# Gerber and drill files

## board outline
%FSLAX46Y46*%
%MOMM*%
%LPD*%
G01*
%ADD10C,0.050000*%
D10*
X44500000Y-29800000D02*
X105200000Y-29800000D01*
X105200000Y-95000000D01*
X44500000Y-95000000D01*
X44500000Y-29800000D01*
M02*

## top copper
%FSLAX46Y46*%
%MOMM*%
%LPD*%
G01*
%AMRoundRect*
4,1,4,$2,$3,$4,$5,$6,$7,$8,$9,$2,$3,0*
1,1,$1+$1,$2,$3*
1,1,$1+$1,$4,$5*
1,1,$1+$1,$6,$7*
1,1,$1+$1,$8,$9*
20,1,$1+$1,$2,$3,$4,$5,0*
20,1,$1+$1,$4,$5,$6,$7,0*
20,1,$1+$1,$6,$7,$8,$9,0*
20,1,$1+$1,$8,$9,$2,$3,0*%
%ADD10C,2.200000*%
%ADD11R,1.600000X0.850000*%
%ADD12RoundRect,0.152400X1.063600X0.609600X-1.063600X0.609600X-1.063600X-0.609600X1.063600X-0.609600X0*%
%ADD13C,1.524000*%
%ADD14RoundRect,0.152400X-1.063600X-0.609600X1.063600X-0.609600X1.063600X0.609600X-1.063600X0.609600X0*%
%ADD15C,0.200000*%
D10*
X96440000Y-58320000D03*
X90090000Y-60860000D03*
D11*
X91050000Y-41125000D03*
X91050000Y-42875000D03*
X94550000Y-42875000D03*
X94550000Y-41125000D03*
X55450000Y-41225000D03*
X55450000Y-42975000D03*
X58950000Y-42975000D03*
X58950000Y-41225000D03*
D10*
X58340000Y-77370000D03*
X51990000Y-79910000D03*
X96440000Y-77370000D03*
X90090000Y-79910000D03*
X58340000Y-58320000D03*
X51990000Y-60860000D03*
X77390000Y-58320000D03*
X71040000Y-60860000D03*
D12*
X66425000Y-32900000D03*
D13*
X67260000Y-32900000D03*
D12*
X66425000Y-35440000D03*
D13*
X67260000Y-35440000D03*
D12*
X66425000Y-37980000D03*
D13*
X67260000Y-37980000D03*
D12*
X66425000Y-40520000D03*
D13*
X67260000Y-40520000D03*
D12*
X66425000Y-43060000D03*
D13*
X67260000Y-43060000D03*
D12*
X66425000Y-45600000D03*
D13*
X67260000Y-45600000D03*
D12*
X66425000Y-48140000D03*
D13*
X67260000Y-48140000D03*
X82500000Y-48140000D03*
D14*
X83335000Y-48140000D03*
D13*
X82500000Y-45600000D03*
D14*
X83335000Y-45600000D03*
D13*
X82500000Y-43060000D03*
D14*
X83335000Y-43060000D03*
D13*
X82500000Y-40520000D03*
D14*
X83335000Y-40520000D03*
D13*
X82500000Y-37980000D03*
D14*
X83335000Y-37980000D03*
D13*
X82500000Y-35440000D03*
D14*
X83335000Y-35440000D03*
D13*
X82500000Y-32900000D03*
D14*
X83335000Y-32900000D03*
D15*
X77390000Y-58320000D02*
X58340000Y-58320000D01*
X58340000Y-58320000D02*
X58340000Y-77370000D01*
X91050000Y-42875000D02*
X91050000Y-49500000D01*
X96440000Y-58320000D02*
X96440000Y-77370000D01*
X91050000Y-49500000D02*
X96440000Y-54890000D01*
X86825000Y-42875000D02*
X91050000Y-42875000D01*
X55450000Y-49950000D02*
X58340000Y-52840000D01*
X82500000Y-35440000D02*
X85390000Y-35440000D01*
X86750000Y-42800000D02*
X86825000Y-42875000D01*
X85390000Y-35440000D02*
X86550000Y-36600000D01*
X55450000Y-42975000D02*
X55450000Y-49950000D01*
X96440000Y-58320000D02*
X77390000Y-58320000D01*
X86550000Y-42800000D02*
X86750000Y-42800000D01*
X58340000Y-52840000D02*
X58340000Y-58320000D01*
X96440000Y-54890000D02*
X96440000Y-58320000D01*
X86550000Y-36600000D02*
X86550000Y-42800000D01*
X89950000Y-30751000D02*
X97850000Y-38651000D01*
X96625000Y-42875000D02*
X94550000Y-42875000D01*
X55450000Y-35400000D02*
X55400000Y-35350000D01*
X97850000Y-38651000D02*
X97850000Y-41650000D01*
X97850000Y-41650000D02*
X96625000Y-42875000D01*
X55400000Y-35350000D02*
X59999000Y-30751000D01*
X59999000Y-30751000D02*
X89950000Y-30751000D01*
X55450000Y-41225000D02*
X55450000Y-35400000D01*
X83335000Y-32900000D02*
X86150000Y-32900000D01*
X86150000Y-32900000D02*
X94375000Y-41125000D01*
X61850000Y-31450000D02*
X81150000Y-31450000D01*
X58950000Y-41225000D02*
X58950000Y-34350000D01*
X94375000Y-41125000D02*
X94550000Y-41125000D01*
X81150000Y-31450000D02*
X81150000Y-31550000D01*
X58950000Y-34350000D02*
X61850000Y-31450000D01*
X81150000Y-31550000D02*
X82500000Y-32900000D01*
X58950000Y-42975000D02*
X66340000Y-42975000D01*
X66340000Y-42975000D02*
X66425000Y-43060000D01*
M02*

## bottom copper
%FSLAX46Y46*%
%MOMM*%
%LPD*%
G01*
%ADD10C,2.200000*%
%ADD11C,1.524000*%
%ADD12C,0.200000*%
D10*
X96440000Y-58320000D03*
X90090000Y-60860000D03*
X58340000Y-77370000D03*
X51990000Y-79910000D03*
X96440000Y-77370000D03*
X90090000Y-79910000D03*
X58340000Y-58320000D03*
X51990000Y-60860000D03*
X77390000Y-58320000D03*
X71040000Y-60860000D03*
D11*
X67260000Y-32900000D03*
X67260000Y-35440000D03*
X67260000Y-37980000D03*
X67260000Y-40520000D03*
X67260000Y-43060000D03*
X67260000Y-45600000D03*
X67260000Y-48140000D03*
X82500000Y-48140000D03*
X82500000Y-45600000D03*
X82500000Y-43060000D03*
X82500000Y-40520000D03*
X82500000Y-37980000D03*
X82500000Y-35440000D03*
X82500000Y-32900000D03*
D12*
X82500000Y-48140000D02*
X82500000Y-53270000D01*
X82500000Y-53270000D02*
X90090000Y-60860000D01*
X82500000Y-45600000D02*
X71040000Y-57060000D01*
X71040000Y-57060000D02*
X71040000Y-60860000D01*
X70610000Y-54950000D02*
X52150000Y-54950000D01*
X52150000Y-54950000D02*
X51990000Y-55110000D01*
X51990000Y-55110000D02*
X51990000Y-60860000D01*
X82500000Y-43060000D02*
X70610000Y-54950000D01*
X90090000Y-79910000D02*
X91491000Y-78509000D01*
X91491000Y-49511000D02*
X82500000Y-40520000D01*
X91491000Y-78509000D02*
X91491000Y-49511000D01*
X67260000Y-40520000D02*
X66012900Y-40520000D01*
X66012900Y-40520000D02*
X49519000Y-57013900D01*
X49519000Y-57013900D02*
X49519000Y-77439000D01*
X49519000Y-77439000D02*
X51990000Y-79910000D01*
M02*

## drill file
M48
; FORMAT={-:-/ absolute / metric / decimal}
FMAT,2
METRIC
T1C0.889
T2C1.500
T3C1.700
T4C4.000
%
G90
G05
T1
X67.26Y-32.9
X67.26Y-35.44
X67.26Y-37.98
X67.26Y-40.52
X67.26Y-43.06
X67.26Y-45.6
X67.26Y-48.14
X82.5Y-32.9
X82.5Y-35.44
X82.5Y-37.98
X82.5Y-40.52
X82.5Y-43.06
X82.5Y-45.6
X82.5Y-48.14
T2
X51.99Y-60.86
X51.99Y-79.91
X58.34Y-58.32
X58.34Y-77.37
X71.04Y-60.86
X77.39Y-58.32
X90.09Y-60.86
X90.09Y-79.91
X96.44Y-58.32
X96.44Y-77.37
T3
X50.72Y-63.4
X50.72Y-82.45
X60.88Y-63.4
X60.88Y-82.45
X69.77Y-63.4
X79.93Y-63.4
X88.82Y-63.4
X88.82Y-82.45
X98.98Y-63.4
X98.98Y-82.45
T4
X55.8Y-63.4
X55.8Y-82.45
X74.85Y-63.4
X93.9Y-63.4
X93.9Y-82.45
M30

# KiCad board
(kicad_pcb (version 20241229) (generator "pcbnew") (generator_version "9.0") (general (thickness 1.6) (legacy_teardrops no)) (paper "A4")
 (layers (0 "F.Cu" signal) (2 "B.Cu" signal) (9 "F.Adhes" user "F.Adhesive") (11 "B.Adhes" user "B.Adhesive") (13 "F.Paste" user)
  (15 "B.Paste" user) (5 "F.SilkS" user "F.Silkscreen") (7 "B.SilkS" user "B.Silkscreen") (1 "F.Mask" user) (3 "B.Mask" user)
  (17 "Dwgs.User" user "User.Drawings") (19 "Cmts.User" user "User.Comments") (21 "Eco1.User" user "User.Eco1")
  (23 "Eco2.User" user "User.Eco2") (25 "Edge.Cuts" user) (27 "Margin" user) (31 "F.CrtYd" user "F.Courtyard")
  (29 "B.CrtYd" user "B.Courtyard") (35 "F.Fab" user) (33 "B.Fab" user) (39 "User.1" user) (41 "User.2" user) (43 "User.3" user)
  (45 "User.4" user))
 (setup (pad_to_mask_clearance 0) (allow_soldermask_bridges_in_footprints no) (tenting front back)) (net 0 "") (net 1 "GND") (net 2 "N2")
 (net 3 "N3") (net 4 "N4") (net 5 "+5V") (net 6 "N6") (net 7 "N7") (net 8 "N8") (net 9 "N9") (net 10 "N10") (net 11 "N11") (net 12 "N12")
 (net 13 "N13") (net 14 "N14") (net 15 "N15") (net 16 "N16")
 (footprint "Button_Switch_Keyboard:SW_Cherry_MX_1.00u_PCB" (layer "F.Cu") (at 96.44 58.32)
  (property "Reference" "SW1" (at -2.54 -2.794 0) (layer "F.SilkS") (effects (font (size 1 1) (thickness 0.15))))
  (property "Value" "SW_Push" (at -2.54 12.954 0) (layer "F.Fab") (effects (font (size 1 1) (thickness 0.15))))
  (pad "" np_thru_hole circle (at -7.62 5.08) (size 1.7 1.7) (drill 1.7) (layers "*.Cu" "*.Mask"))
  (pad "" np_thru_hole circle (at -2.54 5.08) (size 4 4) (drill 4) (layers "*.Cu" "*.Mask"))
  (pad "" np_thru_hole circle (at 2.54 5.08) (size 1.7 1.7) (drill 1.7) (layers "*.Cu" "*.Mask"))
  (pad "1" thru_hole circle (at 0 0) (size 2.2 2.2) (drill 1.5) (layers "*.Cu" "*.Mask") (remove_unused_layers no) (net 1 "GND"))
  (pad "2" thru_hole circle (at -6.35 2.54) (size 2.2 2.2) (drill 1.5) (layers "*.Cu" "*.Mask") (remove_unused_layers no) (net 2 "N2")))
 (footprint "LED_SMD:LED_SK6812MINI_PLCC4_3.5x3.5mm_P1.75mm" (layer "F.Cu") (at 92.8 42)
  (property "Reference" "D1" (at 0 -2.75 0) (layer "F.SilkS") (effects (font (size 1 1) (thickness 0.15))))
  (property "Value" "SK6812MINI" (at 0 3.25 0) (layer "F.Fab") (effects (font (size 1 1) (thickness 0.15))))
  (pad "1" smd rect (at -1.75 -0.875) (size 1.6 0.85) (layers "F.Cu" "F.Mask" "F.Paste") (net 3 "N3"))
  (pad "2" smd rect (at -1.75 0.875) (size 1.6 0.85) (layers "F.Cu" "F.Mask" "F.Paste") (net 1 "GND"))
  (pad "3" smd rect (at 1.75 0.875) (size 1.6 0.85) (layers "F.Cu" "F.Mask" "F.Paste") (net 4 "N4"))
  (pad "4" smd rect (at 1.75 -0.875) (size 1.6 0.85) (layers "F.Cu" "F.Mask" "F.Paste") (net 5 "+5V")))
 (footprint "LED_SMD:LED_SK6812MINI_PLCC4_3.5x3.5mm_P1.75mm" (layer "F.Cu") (at 57.2 42.1)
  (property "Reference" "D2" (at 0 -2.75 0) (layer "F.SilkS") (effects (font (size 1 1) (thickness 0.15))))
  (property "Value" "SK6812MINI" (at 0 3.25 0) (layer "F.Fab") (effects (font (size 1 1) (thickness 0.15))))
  (pad "1" smd rect (at -1.75 -0.875) (size 1.6 0.85) (layers "F.Cu" "F.Mask" "F.Paste") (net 4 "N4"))
  (pad "2" smd rect (at -1.75 0.875) (size 1.6 0.85) (layers "F.Cu" "F.Mask" "F.Paste") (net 1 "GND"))
  (pad "3" smd rect (at 1.75 0.875) (size 1.6 0.85) (layers "F.Cu" "F.Mask" "F.Paste") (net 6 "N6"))
  (pad "4" smd rect (at 1.75 -0.875) (size 1.6 0.85) (layers "F.Cu" "F.Mask" "F.Paste") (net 5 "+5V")))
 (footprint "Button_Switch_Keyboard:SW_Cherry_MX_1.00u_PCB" (layer "F.Cu") (at 58.34 77.37)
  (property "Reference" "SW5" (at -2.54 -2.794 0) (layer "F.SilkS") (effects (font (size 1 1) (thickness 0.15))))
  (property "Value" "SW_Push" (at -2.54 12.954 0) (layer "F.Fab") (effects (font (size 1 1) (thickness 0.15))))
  (pad "" np_thru_hole circle (at -7.62 5.08) (size 1.7 1.7) (drill 1.7) (layers "*.Cu" "*.Mask"))
  (pad "" np_thru_hole circle (at -2.54 5.08) (size 4 4) (drill 4) (layers "*.Cu" "*.Mask"))
  (pad "" np_thru_hole circle (at 2.54 5.08) (size 1.7 1.7) (drill 1.7) (layers "*.Cu" "*.Mask"))
  (pad "1" thru_hole circle (at 0 0) (size 2.2 2.2) (drill 1.5) (layers "*.Cu" "*.Mask") (remove_unused_layers no) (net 1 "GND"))
  (pad "2" thru_hole circle (at -6.35 2.54) (size 2.2 2.2) (drill 1.5) (layers "*.Cu" "*.Mask") (remove_unused_layers no) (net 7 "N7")))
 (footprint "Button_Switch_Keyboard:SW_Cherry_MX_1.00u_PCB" (layer "F.Cu") (at 96.44 77.37)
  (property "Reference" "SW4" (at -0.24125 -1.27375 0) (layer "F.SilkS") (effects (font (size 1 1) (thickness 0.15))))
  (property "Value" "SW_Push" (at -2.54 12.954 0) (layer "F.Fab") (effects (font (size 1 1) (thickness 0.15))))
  (pad "" np_thru_hole circle (at -7.62 5.08) (size 1.7 1.7) (drill 1.7) (layers "*.Cu" "*.Mask"))
  (pad "" np_thru_hole circle (at -2.54 5.08) (size 4 4) (drill 4) (layers "*.Cu" "*.Mask"))
  (pad "" np_thru_hole circle (at 2.54 5.08) (size 1.7 1.7) (drill 1.7) (layers "*.Cu" "*.Mask"))
  (pad "1" thru_hole circle (at 0 0) (size 2.2 2.2) (drill 1.5) (layers "*.Cu" "*.Mask") (remove_unused_layers no) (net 1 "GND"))
  (pad "2" thru_hole circle (at -6.35 2.54) (size 2.2 2.2) (drill 1.5) (layers "*.Cu" "*.Mask") (remove_unused_layers no) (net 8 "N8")))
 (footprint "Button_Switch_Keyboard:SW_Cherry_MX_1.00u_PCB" (layer "F.Cu") (at 58.34 58.32)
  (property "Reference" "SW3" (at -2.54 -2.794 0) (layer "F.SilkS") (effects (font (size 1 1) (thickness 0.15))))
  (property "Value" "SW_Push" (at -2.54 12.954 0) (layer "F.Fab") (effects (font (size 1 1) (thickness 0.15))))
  (pad "" np_thru_hole circle (at -7.62 5.08) (size 1.7 1.7) (drill 1.7) (layers "*.Cu" "*.Mask"))
  (pad "" np_thru_hole circle (at -2.54 5.08) (size 4 4) (drill 4) (layers "*.Cu" "*.Mask"))
  (pad "" np_thru_hole circle (at 2.54 5.08) (size 1.7 1.7) (drill 1.7) (layers "*.Cu" "*.Mask"))
  (pad "1" thru_hole circle (at 0 0) (size 2.2 2.2) (drill 1.5) (layers "*.Cu" "*.Mask") (remove_unused_layers no) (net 1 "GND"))
  (pad "2" thru_hole circle (at -6.35 2.54) (size 2.2 2.2) (drill 1.5) (layers "*.Cu" "*.Mask") (remove_unused_layers no) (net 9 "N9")))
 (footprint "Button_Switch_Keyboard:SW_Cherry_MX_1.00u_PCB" (layer "F.Cu") (at 77.39 58.32)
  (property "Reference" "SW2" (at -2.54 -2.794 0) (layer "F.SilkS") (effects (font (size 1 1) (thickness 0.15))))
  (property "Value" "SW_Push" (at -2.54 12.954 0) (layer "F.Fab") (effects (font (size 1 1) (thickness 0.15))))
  (pad "" np_thru_hole circle (at -7.62 5.08) (size 1.7 1.7) (drill 1.7) (layers "*.Cu" "*.Mask"))
  (pad "" np_thru_hole circle (at -2.54 5.08) (size 4 4) (drill 4) (layers "*.Cu" "*.Mask"))
  (pad "" np_thru_hole circle (at 2.54 5.08) (size 1.7 1.7) (drill 1.7) (layers "*.Cu" "*.Mask"))
  (pad "1" thru_hole circle (at 0 0) (size 2.2 2.2) (drill 1.5) (layers "*.Cu" "*.Mask") (remove_unused_layers no) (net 1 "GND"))
  (pad "2" thru_hole circle (at -6.35 2.54) (size 2.2 2.2) (drill 1.5) (layers "*.Cu" "*.Mask") (remove_unused_layers no) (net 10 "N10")))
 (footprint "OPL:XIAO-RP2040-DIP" (layer "F.Cu") (at 74.88 40.52)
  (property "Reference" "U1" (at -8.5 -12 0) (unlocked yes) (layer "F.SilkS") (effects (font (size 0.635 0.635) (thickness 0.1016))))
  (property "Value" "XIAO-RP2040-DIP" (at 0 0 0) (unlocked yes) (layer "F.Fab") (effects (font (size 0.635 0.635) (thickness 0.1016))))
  (pad "1" smd roundrect (at -8.455 -7.62 180) (size 2.432 1.524) (layers "F.Cu" "F.Mask") (roundrect_rratio 0.1) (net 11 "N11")
   (thermal_bridge_angle 45))
  (pad "1" thru_hole circle (at -7.62 -7.62 180) (size 1.524 1.524) (drill 0.889) (layers "*.Cu" "*.Mask") (remove_unused_layers no)
   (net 11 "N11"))
  (pad "2" smd roundrect (at -8.455 -5.08 180) (size 2.432 1.524) (layers "F.Cu" "F.Mask") (roundrect_rratio 0.1) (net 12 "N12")
   (thermal_bridge_angle 45))
  (pad "2" thru_hole circle (at -7.62 -5.08 180) (size 1.524 1.524) (drill 0.889) (layers "*.Cu" "*.Mask") (remove_unused_layers no)
   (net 12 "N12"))
  (pad "3" smd roundrect (at -8.455 -2.54 180) (size 2.432 1.524) (layers "F.Cu" "F.Mask") (roundrect_rratio 0.1) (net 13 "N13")
   (thermal_bridge_angle 45))
  (pad "3" thru_hole circle (at -7.62 -2.54 180) (size 1.524 1.524) (drill 0.889) (layers "*.Cu" "*.Mask") (remove_unused_layers no)
   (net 13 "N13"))
  (pad "4" smd roundrect (at -8.455 0 180) (size 2.432 1.524) (layers "F.Cu" "F.Mask") (roundrect_rratio 0.1) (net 7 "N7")
   (thermal_bridge_angle 45))
  (pad "4" thru_hole circle (at -7.62 0 180) (size 1.524 1.524) (drill 0.889) (layers "*.Cu" "*.Mask") (remove_unused_layers no)
   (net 7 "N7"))
  (pad "5" smd roundrect (at -8.455 2.54 180) (size 2.432 1.524) (layers "F.Cu" "F.Mask") (roundrect_rratio 0.1) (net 6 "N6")
   (thermal_bridge_angle 45))
  (pad "5" thru_hole circle (at -7.62 2.54 180) (size 1.524 1.524) (drill 0.889) (layers "*.Cu" "*.Mask") (remove_unused_layers no)
   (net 6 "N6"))
  (pad "6" smd roundrect (at -8.455 5.08 180) (size 2.432 1.524) (layers "F.Cu" "F.Mask") (roundrect_rratio 0.1) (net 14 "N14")
   (thermal_bridge_angle 45))
  (pad "6" thru_hole circle (at -7.62 5.08 180) (size 1.524 1.524) (drill 0.889) (layers "*.Cu" "*.Mask") (remove_unused_layers no)
   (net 14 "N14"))
  (pad "7" smd roundrect (at -8.455 7.62 180) (size 2.432 1.524) (layers "F.Cu" "F.Mask") (roundrect_rratio 0.1) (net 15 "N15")
   (thermal_bridge_angle 45))
  (pad "7" thru_hole circle (at -7.62 7.62 180) (size 1.524 1.524) (drill 0.889) (layers "*.Cu" "*.Mask") (remove_unused_layers no)
   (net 15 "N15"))
  (pad "8" thru_hole circle (at 7.62 7.62) (size 1.524 1.524) (drill 0.889) (layers "*.Cu" "*.Mask") (remove_unused_layers no) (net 2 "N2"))
  (pad "8" smd roundrect (at 8.455 7.62) (size 2.432 1.524) (layers "F.Cu" "F.Mask") (roundrect_rratio 0.1) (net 2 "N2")
   (thermal_bridge_angle 45))
  (pad "9" thru_hole circle (at 7.62 5.08) (size 1.524 1.524) (drill 0.889) (layers "*.Cu" "*.Mask") (remove_unused_layers no)
   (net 10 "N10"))
  (pad "9" smd roundrect (at 8.455 5.08) (size 2.432 1.524) (layers "F.Cu" "F.Mask") (roundrect_rratio 0.1) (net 10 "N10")
   (thermal_bridge_angle 45))
  (pad "10" thru_hole circle (at 7.62 2.54) (size 1.524 1.524) (drill 0.889) (layers "*.Cu" "*.Mask") (remove_unused_layers no) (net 9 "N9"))
  (pad "10" smd roundrect (at 8.455 2.54) (size 2.432 1.524) (layers "F.Cu" "F.Mask") (roundrect_rratio 0.1) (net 9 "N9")
   (thermal_bridge_angle 45))
  (pad "11" thru_hole circle (at 7.62 0) (size 1.524 1.524) (drill 0.889) (layers "*.Cu" "*.Mask") (remove_unused_layers no) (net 8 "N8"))
  (pad "11" smd roundrect (at 8.455 0) (size 2.432 1.524) (layers "F.Cu" "F.Mask") (roundrect_rratio 0.1) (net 8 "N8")
   (thermal_bridge_angle 45))
  (pad "12" thru_hole circle (at 7.62 -2.54) (size 1.524 1.524) (drill 0.889) (layers "*.Cu" "*.Mask") (remove_unused_layers no)
   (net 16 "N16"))
  (pad "12" smd roundrect (at 8.455 -2.54) (size 2.432 1.524) (layers "F.Cu" "F.Mask") (roundrect_rratio 0.1) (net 16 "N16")
   (thermal_bridge_angle 45))
  (pad "13" thru_hole circle (at 7.62 -5.08) (size 1.524 1.524) (drill 0.889) (layers "*.Cu" "*.Mask") (remove_unused_layers no)
   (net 1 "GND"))
  (pad "13" smd roundrect (at 8.455 -5.08) (size 2.432 1.524) (layers "F.Cu" "F.Mask") (roundrect_rratio 0.1) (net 1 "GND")
   (thermal_bridge_angle 45))
  (pad "14" thru_hole circle (at 7.62 -7.62) (size 1.524 1.524) (drill 0.889) (layers "*.Cu" "*.Mask") (remove_unused_layers no)
   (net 5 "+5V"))
  (pad "14" smd roundrect (at 8.455 -7.62) (size 2.432 1.524) (layers "F.Cu" "F.Mask") (roundrect_rratio 0.1) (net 5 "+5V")
   (thermal_bridge_angle 45)))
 (gr_rect (start 44.5 29.8) (end 105.2 95) (stroke (width 0.05) (type default)) (fill no) (layer "Edge.Cuts"))
 (segment (start 77.39 58.32) (end 58.34 58.32) (width 0.2) (layer "F.Cu") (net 1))
 (segment (start 58.34 58.32) (end 58.34 77.37) (width 0.2) (layer "F.Cu") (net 1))
 (segment (start 91.05 42.875) (end 91.05 49.5) (width 0.2) (layer "F.Cu") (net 1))
 (segment (start 96.44 58.32) (end 96.44 77.37) (width 0.2) (layer "F.Cu") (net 1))
 (segment (start 91.05 49.5) (end 96.44 54.89) (width 0.2) (layer "F.Cu") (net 1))
 (segment (start 86.825 42.875) (end 91.05 42.875) (width 0.2) (layer "F.Cu") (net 1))
 (segment (start 55.45 49.95) (end 58.34 52.84) (width 0.2) (layer "F.Cu") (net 1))
 (segment (start 82.5 35.44) (end 85.39 35.44) (width 0.2) (layer "F.Cu") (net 1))
 (segment (start 86.75 42.8) (end 86.825 42.875) (width 0.2) (layer "F.Cu") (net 1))
 (segment (start 85.39 35.44) (end 86.55 36.6) (width 0.2) (layer "F.Cu") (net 1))
 (segment (start 55.45 42.975) (end 55.45 49.95) (width 0.2) (layer "F.Cu") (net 1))
 (segment (start 96.44 58.32) (end 77.39 58.32) (width 0.2) (layer "F.Cu") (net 1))
 (segment (start 86.55 42.8) (end 86.75 42.8) (width 0.2) (layer "F.Cu") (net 1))
 (segment (start 58.34 52.84) (end 58.34 58.32) (width 0.2) (layer "F.Cu") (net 1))
 (segment (start 96.44 54.89) (end 96.44 58.32) (width 0.2) (layer "F.Cu") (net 1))
 (segment (start 86.55 36.6) (end 86.55 42.8) (width 0.2) (layer "F.Cu") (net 1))
 (segment (start 89.95 30.751) (end 97.85 38.651) (width 0.2) (layer "F.Cu") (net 4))
 (segment (start 96.625 42.875) (end 94.55 42.875) (width 0.2) (layer "F.Cu") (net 4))
 (segment (start 55.45 35.4) (end 55.4 35.35) (width 0.2) (layer "F.Cu") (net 4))
 (segment (start 97.85 38.651) (end 97.85 41.65) (width 0.2) (layer "F.Cu") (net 4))
 (segment (start 97.85 41.65) (end 96.625 42.875) (width 0.2) (layer "F.Cu") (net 4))
 (segment (start 55.4 35.35) (end 59.999 30.751) (width 0.2) (layer "F.Cu") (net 4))
 (segment (start 59.999 30.751) (end 89.95 30.751) (width 0.2) (layer "F.Cu") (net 4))
 (segment (start 55.45 41.225) (end 55.45 35.4) (width 0.2) (layer "F.Cu") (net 4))
 (segment (start 83.335 32.9) (end 86.15 32.9) (width 0.2) (layer "F.Cu") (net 5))
 (segment (start 86.15 32.9) (end 94.375 41.125) (width 0.2) (layer "F.Cu") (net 5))
 (segment (start 61.85 31.45) (end 81.15 31.45) (width 0.2) (layer "F.Cu") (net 5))
 (segment (start 58.95 41.225) (end 58.95 34.35) (width 0.2) (layer "F.Cu") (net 5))
 (segment (start 94.375 41.125) (end 94.55 41.125) (width 0.2) (layer "F.Cu") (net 5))
 (segment (start 81.15 31.45) (end 81.15 31.55) (width 0.2) (layer "F.Cu") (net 5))
 (segment (start 58.95 34.35) (end 61.85 31.45) (width 0.2) (layer "F.Cu") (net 5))
 (segment (start 81.15 31.55) (end 82.5 32.9) (width 0.2) (layer "F.Cu") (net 5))
 (segment (start 58.95 42.975) (end 66.34 42.975) (width 0.2) (layer "F.Cu") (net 6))
 (segment (start 66.34 42.975) (end 66.425 43.06) (width 0.2) (layer "F.Cu") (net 6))
 (segment (start 82.5 48.14) (end 82.5 53.27) (width 0.2) (layer "B.Cu") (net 2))
 (segment (start 82.5 53.27) (end 90.09 60.86) (width 0.2) (layer "B.Cu") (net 2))
 (segment (start 82.5 45.6) (end 71.04 57.06) (width 0.2) (layer "B.Cu") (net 10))
 (segment (start 71.04 57.06) (end 71.04 60.86) (width 0.2) (layer "B.Cu") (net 10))
 (segment (start 70.61 54.95) (end 52.15 54.95) (width 0.2) (layer "B.Cu") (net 9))
 (segment (start 52.15 54.95) (end 51.99 55.11) (width 0.2) (layer "B.Cu") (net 9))
 (segment (start 51.99 55.11) (end 51.99 60.86) (width 0.2) (layer "B.Cu") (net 9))
 (segment (start 82.5 43.06) (end 70.61 54.95) (width 0.2) (layer "B.Cu") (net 9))
 (segment (start 90.09 79.91) (end 91.491 78.509) (width 0.2) (layer "B.Cu") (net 8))
 (segment (start 91.491 49.511) (end 82.5 40.52) (width 0.2) (layer "B.Cu") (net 8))
 (segment (start 91.491 78.509) (end 91.491 49.511) (width 0.2) (layer "B.Cu") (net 8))
 (segment (start 67.26 40.52) (end 66.0129 40.52) (width 0.2) (layer "B.Cu") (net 7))
 (segment (start 66.0129 40.52) (end 49.519 57.0139) (width 0.2) (layer "B.Cu") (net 7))
 (segment (start 49.519 57.0139) (end 49.519 77.439) (width 0.2) (layer "B.Cu") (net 7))
 (segment (start 49.519 77.439) (end 51.99 79.91) (width 0.2) (layer "B.Cu") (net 7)))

